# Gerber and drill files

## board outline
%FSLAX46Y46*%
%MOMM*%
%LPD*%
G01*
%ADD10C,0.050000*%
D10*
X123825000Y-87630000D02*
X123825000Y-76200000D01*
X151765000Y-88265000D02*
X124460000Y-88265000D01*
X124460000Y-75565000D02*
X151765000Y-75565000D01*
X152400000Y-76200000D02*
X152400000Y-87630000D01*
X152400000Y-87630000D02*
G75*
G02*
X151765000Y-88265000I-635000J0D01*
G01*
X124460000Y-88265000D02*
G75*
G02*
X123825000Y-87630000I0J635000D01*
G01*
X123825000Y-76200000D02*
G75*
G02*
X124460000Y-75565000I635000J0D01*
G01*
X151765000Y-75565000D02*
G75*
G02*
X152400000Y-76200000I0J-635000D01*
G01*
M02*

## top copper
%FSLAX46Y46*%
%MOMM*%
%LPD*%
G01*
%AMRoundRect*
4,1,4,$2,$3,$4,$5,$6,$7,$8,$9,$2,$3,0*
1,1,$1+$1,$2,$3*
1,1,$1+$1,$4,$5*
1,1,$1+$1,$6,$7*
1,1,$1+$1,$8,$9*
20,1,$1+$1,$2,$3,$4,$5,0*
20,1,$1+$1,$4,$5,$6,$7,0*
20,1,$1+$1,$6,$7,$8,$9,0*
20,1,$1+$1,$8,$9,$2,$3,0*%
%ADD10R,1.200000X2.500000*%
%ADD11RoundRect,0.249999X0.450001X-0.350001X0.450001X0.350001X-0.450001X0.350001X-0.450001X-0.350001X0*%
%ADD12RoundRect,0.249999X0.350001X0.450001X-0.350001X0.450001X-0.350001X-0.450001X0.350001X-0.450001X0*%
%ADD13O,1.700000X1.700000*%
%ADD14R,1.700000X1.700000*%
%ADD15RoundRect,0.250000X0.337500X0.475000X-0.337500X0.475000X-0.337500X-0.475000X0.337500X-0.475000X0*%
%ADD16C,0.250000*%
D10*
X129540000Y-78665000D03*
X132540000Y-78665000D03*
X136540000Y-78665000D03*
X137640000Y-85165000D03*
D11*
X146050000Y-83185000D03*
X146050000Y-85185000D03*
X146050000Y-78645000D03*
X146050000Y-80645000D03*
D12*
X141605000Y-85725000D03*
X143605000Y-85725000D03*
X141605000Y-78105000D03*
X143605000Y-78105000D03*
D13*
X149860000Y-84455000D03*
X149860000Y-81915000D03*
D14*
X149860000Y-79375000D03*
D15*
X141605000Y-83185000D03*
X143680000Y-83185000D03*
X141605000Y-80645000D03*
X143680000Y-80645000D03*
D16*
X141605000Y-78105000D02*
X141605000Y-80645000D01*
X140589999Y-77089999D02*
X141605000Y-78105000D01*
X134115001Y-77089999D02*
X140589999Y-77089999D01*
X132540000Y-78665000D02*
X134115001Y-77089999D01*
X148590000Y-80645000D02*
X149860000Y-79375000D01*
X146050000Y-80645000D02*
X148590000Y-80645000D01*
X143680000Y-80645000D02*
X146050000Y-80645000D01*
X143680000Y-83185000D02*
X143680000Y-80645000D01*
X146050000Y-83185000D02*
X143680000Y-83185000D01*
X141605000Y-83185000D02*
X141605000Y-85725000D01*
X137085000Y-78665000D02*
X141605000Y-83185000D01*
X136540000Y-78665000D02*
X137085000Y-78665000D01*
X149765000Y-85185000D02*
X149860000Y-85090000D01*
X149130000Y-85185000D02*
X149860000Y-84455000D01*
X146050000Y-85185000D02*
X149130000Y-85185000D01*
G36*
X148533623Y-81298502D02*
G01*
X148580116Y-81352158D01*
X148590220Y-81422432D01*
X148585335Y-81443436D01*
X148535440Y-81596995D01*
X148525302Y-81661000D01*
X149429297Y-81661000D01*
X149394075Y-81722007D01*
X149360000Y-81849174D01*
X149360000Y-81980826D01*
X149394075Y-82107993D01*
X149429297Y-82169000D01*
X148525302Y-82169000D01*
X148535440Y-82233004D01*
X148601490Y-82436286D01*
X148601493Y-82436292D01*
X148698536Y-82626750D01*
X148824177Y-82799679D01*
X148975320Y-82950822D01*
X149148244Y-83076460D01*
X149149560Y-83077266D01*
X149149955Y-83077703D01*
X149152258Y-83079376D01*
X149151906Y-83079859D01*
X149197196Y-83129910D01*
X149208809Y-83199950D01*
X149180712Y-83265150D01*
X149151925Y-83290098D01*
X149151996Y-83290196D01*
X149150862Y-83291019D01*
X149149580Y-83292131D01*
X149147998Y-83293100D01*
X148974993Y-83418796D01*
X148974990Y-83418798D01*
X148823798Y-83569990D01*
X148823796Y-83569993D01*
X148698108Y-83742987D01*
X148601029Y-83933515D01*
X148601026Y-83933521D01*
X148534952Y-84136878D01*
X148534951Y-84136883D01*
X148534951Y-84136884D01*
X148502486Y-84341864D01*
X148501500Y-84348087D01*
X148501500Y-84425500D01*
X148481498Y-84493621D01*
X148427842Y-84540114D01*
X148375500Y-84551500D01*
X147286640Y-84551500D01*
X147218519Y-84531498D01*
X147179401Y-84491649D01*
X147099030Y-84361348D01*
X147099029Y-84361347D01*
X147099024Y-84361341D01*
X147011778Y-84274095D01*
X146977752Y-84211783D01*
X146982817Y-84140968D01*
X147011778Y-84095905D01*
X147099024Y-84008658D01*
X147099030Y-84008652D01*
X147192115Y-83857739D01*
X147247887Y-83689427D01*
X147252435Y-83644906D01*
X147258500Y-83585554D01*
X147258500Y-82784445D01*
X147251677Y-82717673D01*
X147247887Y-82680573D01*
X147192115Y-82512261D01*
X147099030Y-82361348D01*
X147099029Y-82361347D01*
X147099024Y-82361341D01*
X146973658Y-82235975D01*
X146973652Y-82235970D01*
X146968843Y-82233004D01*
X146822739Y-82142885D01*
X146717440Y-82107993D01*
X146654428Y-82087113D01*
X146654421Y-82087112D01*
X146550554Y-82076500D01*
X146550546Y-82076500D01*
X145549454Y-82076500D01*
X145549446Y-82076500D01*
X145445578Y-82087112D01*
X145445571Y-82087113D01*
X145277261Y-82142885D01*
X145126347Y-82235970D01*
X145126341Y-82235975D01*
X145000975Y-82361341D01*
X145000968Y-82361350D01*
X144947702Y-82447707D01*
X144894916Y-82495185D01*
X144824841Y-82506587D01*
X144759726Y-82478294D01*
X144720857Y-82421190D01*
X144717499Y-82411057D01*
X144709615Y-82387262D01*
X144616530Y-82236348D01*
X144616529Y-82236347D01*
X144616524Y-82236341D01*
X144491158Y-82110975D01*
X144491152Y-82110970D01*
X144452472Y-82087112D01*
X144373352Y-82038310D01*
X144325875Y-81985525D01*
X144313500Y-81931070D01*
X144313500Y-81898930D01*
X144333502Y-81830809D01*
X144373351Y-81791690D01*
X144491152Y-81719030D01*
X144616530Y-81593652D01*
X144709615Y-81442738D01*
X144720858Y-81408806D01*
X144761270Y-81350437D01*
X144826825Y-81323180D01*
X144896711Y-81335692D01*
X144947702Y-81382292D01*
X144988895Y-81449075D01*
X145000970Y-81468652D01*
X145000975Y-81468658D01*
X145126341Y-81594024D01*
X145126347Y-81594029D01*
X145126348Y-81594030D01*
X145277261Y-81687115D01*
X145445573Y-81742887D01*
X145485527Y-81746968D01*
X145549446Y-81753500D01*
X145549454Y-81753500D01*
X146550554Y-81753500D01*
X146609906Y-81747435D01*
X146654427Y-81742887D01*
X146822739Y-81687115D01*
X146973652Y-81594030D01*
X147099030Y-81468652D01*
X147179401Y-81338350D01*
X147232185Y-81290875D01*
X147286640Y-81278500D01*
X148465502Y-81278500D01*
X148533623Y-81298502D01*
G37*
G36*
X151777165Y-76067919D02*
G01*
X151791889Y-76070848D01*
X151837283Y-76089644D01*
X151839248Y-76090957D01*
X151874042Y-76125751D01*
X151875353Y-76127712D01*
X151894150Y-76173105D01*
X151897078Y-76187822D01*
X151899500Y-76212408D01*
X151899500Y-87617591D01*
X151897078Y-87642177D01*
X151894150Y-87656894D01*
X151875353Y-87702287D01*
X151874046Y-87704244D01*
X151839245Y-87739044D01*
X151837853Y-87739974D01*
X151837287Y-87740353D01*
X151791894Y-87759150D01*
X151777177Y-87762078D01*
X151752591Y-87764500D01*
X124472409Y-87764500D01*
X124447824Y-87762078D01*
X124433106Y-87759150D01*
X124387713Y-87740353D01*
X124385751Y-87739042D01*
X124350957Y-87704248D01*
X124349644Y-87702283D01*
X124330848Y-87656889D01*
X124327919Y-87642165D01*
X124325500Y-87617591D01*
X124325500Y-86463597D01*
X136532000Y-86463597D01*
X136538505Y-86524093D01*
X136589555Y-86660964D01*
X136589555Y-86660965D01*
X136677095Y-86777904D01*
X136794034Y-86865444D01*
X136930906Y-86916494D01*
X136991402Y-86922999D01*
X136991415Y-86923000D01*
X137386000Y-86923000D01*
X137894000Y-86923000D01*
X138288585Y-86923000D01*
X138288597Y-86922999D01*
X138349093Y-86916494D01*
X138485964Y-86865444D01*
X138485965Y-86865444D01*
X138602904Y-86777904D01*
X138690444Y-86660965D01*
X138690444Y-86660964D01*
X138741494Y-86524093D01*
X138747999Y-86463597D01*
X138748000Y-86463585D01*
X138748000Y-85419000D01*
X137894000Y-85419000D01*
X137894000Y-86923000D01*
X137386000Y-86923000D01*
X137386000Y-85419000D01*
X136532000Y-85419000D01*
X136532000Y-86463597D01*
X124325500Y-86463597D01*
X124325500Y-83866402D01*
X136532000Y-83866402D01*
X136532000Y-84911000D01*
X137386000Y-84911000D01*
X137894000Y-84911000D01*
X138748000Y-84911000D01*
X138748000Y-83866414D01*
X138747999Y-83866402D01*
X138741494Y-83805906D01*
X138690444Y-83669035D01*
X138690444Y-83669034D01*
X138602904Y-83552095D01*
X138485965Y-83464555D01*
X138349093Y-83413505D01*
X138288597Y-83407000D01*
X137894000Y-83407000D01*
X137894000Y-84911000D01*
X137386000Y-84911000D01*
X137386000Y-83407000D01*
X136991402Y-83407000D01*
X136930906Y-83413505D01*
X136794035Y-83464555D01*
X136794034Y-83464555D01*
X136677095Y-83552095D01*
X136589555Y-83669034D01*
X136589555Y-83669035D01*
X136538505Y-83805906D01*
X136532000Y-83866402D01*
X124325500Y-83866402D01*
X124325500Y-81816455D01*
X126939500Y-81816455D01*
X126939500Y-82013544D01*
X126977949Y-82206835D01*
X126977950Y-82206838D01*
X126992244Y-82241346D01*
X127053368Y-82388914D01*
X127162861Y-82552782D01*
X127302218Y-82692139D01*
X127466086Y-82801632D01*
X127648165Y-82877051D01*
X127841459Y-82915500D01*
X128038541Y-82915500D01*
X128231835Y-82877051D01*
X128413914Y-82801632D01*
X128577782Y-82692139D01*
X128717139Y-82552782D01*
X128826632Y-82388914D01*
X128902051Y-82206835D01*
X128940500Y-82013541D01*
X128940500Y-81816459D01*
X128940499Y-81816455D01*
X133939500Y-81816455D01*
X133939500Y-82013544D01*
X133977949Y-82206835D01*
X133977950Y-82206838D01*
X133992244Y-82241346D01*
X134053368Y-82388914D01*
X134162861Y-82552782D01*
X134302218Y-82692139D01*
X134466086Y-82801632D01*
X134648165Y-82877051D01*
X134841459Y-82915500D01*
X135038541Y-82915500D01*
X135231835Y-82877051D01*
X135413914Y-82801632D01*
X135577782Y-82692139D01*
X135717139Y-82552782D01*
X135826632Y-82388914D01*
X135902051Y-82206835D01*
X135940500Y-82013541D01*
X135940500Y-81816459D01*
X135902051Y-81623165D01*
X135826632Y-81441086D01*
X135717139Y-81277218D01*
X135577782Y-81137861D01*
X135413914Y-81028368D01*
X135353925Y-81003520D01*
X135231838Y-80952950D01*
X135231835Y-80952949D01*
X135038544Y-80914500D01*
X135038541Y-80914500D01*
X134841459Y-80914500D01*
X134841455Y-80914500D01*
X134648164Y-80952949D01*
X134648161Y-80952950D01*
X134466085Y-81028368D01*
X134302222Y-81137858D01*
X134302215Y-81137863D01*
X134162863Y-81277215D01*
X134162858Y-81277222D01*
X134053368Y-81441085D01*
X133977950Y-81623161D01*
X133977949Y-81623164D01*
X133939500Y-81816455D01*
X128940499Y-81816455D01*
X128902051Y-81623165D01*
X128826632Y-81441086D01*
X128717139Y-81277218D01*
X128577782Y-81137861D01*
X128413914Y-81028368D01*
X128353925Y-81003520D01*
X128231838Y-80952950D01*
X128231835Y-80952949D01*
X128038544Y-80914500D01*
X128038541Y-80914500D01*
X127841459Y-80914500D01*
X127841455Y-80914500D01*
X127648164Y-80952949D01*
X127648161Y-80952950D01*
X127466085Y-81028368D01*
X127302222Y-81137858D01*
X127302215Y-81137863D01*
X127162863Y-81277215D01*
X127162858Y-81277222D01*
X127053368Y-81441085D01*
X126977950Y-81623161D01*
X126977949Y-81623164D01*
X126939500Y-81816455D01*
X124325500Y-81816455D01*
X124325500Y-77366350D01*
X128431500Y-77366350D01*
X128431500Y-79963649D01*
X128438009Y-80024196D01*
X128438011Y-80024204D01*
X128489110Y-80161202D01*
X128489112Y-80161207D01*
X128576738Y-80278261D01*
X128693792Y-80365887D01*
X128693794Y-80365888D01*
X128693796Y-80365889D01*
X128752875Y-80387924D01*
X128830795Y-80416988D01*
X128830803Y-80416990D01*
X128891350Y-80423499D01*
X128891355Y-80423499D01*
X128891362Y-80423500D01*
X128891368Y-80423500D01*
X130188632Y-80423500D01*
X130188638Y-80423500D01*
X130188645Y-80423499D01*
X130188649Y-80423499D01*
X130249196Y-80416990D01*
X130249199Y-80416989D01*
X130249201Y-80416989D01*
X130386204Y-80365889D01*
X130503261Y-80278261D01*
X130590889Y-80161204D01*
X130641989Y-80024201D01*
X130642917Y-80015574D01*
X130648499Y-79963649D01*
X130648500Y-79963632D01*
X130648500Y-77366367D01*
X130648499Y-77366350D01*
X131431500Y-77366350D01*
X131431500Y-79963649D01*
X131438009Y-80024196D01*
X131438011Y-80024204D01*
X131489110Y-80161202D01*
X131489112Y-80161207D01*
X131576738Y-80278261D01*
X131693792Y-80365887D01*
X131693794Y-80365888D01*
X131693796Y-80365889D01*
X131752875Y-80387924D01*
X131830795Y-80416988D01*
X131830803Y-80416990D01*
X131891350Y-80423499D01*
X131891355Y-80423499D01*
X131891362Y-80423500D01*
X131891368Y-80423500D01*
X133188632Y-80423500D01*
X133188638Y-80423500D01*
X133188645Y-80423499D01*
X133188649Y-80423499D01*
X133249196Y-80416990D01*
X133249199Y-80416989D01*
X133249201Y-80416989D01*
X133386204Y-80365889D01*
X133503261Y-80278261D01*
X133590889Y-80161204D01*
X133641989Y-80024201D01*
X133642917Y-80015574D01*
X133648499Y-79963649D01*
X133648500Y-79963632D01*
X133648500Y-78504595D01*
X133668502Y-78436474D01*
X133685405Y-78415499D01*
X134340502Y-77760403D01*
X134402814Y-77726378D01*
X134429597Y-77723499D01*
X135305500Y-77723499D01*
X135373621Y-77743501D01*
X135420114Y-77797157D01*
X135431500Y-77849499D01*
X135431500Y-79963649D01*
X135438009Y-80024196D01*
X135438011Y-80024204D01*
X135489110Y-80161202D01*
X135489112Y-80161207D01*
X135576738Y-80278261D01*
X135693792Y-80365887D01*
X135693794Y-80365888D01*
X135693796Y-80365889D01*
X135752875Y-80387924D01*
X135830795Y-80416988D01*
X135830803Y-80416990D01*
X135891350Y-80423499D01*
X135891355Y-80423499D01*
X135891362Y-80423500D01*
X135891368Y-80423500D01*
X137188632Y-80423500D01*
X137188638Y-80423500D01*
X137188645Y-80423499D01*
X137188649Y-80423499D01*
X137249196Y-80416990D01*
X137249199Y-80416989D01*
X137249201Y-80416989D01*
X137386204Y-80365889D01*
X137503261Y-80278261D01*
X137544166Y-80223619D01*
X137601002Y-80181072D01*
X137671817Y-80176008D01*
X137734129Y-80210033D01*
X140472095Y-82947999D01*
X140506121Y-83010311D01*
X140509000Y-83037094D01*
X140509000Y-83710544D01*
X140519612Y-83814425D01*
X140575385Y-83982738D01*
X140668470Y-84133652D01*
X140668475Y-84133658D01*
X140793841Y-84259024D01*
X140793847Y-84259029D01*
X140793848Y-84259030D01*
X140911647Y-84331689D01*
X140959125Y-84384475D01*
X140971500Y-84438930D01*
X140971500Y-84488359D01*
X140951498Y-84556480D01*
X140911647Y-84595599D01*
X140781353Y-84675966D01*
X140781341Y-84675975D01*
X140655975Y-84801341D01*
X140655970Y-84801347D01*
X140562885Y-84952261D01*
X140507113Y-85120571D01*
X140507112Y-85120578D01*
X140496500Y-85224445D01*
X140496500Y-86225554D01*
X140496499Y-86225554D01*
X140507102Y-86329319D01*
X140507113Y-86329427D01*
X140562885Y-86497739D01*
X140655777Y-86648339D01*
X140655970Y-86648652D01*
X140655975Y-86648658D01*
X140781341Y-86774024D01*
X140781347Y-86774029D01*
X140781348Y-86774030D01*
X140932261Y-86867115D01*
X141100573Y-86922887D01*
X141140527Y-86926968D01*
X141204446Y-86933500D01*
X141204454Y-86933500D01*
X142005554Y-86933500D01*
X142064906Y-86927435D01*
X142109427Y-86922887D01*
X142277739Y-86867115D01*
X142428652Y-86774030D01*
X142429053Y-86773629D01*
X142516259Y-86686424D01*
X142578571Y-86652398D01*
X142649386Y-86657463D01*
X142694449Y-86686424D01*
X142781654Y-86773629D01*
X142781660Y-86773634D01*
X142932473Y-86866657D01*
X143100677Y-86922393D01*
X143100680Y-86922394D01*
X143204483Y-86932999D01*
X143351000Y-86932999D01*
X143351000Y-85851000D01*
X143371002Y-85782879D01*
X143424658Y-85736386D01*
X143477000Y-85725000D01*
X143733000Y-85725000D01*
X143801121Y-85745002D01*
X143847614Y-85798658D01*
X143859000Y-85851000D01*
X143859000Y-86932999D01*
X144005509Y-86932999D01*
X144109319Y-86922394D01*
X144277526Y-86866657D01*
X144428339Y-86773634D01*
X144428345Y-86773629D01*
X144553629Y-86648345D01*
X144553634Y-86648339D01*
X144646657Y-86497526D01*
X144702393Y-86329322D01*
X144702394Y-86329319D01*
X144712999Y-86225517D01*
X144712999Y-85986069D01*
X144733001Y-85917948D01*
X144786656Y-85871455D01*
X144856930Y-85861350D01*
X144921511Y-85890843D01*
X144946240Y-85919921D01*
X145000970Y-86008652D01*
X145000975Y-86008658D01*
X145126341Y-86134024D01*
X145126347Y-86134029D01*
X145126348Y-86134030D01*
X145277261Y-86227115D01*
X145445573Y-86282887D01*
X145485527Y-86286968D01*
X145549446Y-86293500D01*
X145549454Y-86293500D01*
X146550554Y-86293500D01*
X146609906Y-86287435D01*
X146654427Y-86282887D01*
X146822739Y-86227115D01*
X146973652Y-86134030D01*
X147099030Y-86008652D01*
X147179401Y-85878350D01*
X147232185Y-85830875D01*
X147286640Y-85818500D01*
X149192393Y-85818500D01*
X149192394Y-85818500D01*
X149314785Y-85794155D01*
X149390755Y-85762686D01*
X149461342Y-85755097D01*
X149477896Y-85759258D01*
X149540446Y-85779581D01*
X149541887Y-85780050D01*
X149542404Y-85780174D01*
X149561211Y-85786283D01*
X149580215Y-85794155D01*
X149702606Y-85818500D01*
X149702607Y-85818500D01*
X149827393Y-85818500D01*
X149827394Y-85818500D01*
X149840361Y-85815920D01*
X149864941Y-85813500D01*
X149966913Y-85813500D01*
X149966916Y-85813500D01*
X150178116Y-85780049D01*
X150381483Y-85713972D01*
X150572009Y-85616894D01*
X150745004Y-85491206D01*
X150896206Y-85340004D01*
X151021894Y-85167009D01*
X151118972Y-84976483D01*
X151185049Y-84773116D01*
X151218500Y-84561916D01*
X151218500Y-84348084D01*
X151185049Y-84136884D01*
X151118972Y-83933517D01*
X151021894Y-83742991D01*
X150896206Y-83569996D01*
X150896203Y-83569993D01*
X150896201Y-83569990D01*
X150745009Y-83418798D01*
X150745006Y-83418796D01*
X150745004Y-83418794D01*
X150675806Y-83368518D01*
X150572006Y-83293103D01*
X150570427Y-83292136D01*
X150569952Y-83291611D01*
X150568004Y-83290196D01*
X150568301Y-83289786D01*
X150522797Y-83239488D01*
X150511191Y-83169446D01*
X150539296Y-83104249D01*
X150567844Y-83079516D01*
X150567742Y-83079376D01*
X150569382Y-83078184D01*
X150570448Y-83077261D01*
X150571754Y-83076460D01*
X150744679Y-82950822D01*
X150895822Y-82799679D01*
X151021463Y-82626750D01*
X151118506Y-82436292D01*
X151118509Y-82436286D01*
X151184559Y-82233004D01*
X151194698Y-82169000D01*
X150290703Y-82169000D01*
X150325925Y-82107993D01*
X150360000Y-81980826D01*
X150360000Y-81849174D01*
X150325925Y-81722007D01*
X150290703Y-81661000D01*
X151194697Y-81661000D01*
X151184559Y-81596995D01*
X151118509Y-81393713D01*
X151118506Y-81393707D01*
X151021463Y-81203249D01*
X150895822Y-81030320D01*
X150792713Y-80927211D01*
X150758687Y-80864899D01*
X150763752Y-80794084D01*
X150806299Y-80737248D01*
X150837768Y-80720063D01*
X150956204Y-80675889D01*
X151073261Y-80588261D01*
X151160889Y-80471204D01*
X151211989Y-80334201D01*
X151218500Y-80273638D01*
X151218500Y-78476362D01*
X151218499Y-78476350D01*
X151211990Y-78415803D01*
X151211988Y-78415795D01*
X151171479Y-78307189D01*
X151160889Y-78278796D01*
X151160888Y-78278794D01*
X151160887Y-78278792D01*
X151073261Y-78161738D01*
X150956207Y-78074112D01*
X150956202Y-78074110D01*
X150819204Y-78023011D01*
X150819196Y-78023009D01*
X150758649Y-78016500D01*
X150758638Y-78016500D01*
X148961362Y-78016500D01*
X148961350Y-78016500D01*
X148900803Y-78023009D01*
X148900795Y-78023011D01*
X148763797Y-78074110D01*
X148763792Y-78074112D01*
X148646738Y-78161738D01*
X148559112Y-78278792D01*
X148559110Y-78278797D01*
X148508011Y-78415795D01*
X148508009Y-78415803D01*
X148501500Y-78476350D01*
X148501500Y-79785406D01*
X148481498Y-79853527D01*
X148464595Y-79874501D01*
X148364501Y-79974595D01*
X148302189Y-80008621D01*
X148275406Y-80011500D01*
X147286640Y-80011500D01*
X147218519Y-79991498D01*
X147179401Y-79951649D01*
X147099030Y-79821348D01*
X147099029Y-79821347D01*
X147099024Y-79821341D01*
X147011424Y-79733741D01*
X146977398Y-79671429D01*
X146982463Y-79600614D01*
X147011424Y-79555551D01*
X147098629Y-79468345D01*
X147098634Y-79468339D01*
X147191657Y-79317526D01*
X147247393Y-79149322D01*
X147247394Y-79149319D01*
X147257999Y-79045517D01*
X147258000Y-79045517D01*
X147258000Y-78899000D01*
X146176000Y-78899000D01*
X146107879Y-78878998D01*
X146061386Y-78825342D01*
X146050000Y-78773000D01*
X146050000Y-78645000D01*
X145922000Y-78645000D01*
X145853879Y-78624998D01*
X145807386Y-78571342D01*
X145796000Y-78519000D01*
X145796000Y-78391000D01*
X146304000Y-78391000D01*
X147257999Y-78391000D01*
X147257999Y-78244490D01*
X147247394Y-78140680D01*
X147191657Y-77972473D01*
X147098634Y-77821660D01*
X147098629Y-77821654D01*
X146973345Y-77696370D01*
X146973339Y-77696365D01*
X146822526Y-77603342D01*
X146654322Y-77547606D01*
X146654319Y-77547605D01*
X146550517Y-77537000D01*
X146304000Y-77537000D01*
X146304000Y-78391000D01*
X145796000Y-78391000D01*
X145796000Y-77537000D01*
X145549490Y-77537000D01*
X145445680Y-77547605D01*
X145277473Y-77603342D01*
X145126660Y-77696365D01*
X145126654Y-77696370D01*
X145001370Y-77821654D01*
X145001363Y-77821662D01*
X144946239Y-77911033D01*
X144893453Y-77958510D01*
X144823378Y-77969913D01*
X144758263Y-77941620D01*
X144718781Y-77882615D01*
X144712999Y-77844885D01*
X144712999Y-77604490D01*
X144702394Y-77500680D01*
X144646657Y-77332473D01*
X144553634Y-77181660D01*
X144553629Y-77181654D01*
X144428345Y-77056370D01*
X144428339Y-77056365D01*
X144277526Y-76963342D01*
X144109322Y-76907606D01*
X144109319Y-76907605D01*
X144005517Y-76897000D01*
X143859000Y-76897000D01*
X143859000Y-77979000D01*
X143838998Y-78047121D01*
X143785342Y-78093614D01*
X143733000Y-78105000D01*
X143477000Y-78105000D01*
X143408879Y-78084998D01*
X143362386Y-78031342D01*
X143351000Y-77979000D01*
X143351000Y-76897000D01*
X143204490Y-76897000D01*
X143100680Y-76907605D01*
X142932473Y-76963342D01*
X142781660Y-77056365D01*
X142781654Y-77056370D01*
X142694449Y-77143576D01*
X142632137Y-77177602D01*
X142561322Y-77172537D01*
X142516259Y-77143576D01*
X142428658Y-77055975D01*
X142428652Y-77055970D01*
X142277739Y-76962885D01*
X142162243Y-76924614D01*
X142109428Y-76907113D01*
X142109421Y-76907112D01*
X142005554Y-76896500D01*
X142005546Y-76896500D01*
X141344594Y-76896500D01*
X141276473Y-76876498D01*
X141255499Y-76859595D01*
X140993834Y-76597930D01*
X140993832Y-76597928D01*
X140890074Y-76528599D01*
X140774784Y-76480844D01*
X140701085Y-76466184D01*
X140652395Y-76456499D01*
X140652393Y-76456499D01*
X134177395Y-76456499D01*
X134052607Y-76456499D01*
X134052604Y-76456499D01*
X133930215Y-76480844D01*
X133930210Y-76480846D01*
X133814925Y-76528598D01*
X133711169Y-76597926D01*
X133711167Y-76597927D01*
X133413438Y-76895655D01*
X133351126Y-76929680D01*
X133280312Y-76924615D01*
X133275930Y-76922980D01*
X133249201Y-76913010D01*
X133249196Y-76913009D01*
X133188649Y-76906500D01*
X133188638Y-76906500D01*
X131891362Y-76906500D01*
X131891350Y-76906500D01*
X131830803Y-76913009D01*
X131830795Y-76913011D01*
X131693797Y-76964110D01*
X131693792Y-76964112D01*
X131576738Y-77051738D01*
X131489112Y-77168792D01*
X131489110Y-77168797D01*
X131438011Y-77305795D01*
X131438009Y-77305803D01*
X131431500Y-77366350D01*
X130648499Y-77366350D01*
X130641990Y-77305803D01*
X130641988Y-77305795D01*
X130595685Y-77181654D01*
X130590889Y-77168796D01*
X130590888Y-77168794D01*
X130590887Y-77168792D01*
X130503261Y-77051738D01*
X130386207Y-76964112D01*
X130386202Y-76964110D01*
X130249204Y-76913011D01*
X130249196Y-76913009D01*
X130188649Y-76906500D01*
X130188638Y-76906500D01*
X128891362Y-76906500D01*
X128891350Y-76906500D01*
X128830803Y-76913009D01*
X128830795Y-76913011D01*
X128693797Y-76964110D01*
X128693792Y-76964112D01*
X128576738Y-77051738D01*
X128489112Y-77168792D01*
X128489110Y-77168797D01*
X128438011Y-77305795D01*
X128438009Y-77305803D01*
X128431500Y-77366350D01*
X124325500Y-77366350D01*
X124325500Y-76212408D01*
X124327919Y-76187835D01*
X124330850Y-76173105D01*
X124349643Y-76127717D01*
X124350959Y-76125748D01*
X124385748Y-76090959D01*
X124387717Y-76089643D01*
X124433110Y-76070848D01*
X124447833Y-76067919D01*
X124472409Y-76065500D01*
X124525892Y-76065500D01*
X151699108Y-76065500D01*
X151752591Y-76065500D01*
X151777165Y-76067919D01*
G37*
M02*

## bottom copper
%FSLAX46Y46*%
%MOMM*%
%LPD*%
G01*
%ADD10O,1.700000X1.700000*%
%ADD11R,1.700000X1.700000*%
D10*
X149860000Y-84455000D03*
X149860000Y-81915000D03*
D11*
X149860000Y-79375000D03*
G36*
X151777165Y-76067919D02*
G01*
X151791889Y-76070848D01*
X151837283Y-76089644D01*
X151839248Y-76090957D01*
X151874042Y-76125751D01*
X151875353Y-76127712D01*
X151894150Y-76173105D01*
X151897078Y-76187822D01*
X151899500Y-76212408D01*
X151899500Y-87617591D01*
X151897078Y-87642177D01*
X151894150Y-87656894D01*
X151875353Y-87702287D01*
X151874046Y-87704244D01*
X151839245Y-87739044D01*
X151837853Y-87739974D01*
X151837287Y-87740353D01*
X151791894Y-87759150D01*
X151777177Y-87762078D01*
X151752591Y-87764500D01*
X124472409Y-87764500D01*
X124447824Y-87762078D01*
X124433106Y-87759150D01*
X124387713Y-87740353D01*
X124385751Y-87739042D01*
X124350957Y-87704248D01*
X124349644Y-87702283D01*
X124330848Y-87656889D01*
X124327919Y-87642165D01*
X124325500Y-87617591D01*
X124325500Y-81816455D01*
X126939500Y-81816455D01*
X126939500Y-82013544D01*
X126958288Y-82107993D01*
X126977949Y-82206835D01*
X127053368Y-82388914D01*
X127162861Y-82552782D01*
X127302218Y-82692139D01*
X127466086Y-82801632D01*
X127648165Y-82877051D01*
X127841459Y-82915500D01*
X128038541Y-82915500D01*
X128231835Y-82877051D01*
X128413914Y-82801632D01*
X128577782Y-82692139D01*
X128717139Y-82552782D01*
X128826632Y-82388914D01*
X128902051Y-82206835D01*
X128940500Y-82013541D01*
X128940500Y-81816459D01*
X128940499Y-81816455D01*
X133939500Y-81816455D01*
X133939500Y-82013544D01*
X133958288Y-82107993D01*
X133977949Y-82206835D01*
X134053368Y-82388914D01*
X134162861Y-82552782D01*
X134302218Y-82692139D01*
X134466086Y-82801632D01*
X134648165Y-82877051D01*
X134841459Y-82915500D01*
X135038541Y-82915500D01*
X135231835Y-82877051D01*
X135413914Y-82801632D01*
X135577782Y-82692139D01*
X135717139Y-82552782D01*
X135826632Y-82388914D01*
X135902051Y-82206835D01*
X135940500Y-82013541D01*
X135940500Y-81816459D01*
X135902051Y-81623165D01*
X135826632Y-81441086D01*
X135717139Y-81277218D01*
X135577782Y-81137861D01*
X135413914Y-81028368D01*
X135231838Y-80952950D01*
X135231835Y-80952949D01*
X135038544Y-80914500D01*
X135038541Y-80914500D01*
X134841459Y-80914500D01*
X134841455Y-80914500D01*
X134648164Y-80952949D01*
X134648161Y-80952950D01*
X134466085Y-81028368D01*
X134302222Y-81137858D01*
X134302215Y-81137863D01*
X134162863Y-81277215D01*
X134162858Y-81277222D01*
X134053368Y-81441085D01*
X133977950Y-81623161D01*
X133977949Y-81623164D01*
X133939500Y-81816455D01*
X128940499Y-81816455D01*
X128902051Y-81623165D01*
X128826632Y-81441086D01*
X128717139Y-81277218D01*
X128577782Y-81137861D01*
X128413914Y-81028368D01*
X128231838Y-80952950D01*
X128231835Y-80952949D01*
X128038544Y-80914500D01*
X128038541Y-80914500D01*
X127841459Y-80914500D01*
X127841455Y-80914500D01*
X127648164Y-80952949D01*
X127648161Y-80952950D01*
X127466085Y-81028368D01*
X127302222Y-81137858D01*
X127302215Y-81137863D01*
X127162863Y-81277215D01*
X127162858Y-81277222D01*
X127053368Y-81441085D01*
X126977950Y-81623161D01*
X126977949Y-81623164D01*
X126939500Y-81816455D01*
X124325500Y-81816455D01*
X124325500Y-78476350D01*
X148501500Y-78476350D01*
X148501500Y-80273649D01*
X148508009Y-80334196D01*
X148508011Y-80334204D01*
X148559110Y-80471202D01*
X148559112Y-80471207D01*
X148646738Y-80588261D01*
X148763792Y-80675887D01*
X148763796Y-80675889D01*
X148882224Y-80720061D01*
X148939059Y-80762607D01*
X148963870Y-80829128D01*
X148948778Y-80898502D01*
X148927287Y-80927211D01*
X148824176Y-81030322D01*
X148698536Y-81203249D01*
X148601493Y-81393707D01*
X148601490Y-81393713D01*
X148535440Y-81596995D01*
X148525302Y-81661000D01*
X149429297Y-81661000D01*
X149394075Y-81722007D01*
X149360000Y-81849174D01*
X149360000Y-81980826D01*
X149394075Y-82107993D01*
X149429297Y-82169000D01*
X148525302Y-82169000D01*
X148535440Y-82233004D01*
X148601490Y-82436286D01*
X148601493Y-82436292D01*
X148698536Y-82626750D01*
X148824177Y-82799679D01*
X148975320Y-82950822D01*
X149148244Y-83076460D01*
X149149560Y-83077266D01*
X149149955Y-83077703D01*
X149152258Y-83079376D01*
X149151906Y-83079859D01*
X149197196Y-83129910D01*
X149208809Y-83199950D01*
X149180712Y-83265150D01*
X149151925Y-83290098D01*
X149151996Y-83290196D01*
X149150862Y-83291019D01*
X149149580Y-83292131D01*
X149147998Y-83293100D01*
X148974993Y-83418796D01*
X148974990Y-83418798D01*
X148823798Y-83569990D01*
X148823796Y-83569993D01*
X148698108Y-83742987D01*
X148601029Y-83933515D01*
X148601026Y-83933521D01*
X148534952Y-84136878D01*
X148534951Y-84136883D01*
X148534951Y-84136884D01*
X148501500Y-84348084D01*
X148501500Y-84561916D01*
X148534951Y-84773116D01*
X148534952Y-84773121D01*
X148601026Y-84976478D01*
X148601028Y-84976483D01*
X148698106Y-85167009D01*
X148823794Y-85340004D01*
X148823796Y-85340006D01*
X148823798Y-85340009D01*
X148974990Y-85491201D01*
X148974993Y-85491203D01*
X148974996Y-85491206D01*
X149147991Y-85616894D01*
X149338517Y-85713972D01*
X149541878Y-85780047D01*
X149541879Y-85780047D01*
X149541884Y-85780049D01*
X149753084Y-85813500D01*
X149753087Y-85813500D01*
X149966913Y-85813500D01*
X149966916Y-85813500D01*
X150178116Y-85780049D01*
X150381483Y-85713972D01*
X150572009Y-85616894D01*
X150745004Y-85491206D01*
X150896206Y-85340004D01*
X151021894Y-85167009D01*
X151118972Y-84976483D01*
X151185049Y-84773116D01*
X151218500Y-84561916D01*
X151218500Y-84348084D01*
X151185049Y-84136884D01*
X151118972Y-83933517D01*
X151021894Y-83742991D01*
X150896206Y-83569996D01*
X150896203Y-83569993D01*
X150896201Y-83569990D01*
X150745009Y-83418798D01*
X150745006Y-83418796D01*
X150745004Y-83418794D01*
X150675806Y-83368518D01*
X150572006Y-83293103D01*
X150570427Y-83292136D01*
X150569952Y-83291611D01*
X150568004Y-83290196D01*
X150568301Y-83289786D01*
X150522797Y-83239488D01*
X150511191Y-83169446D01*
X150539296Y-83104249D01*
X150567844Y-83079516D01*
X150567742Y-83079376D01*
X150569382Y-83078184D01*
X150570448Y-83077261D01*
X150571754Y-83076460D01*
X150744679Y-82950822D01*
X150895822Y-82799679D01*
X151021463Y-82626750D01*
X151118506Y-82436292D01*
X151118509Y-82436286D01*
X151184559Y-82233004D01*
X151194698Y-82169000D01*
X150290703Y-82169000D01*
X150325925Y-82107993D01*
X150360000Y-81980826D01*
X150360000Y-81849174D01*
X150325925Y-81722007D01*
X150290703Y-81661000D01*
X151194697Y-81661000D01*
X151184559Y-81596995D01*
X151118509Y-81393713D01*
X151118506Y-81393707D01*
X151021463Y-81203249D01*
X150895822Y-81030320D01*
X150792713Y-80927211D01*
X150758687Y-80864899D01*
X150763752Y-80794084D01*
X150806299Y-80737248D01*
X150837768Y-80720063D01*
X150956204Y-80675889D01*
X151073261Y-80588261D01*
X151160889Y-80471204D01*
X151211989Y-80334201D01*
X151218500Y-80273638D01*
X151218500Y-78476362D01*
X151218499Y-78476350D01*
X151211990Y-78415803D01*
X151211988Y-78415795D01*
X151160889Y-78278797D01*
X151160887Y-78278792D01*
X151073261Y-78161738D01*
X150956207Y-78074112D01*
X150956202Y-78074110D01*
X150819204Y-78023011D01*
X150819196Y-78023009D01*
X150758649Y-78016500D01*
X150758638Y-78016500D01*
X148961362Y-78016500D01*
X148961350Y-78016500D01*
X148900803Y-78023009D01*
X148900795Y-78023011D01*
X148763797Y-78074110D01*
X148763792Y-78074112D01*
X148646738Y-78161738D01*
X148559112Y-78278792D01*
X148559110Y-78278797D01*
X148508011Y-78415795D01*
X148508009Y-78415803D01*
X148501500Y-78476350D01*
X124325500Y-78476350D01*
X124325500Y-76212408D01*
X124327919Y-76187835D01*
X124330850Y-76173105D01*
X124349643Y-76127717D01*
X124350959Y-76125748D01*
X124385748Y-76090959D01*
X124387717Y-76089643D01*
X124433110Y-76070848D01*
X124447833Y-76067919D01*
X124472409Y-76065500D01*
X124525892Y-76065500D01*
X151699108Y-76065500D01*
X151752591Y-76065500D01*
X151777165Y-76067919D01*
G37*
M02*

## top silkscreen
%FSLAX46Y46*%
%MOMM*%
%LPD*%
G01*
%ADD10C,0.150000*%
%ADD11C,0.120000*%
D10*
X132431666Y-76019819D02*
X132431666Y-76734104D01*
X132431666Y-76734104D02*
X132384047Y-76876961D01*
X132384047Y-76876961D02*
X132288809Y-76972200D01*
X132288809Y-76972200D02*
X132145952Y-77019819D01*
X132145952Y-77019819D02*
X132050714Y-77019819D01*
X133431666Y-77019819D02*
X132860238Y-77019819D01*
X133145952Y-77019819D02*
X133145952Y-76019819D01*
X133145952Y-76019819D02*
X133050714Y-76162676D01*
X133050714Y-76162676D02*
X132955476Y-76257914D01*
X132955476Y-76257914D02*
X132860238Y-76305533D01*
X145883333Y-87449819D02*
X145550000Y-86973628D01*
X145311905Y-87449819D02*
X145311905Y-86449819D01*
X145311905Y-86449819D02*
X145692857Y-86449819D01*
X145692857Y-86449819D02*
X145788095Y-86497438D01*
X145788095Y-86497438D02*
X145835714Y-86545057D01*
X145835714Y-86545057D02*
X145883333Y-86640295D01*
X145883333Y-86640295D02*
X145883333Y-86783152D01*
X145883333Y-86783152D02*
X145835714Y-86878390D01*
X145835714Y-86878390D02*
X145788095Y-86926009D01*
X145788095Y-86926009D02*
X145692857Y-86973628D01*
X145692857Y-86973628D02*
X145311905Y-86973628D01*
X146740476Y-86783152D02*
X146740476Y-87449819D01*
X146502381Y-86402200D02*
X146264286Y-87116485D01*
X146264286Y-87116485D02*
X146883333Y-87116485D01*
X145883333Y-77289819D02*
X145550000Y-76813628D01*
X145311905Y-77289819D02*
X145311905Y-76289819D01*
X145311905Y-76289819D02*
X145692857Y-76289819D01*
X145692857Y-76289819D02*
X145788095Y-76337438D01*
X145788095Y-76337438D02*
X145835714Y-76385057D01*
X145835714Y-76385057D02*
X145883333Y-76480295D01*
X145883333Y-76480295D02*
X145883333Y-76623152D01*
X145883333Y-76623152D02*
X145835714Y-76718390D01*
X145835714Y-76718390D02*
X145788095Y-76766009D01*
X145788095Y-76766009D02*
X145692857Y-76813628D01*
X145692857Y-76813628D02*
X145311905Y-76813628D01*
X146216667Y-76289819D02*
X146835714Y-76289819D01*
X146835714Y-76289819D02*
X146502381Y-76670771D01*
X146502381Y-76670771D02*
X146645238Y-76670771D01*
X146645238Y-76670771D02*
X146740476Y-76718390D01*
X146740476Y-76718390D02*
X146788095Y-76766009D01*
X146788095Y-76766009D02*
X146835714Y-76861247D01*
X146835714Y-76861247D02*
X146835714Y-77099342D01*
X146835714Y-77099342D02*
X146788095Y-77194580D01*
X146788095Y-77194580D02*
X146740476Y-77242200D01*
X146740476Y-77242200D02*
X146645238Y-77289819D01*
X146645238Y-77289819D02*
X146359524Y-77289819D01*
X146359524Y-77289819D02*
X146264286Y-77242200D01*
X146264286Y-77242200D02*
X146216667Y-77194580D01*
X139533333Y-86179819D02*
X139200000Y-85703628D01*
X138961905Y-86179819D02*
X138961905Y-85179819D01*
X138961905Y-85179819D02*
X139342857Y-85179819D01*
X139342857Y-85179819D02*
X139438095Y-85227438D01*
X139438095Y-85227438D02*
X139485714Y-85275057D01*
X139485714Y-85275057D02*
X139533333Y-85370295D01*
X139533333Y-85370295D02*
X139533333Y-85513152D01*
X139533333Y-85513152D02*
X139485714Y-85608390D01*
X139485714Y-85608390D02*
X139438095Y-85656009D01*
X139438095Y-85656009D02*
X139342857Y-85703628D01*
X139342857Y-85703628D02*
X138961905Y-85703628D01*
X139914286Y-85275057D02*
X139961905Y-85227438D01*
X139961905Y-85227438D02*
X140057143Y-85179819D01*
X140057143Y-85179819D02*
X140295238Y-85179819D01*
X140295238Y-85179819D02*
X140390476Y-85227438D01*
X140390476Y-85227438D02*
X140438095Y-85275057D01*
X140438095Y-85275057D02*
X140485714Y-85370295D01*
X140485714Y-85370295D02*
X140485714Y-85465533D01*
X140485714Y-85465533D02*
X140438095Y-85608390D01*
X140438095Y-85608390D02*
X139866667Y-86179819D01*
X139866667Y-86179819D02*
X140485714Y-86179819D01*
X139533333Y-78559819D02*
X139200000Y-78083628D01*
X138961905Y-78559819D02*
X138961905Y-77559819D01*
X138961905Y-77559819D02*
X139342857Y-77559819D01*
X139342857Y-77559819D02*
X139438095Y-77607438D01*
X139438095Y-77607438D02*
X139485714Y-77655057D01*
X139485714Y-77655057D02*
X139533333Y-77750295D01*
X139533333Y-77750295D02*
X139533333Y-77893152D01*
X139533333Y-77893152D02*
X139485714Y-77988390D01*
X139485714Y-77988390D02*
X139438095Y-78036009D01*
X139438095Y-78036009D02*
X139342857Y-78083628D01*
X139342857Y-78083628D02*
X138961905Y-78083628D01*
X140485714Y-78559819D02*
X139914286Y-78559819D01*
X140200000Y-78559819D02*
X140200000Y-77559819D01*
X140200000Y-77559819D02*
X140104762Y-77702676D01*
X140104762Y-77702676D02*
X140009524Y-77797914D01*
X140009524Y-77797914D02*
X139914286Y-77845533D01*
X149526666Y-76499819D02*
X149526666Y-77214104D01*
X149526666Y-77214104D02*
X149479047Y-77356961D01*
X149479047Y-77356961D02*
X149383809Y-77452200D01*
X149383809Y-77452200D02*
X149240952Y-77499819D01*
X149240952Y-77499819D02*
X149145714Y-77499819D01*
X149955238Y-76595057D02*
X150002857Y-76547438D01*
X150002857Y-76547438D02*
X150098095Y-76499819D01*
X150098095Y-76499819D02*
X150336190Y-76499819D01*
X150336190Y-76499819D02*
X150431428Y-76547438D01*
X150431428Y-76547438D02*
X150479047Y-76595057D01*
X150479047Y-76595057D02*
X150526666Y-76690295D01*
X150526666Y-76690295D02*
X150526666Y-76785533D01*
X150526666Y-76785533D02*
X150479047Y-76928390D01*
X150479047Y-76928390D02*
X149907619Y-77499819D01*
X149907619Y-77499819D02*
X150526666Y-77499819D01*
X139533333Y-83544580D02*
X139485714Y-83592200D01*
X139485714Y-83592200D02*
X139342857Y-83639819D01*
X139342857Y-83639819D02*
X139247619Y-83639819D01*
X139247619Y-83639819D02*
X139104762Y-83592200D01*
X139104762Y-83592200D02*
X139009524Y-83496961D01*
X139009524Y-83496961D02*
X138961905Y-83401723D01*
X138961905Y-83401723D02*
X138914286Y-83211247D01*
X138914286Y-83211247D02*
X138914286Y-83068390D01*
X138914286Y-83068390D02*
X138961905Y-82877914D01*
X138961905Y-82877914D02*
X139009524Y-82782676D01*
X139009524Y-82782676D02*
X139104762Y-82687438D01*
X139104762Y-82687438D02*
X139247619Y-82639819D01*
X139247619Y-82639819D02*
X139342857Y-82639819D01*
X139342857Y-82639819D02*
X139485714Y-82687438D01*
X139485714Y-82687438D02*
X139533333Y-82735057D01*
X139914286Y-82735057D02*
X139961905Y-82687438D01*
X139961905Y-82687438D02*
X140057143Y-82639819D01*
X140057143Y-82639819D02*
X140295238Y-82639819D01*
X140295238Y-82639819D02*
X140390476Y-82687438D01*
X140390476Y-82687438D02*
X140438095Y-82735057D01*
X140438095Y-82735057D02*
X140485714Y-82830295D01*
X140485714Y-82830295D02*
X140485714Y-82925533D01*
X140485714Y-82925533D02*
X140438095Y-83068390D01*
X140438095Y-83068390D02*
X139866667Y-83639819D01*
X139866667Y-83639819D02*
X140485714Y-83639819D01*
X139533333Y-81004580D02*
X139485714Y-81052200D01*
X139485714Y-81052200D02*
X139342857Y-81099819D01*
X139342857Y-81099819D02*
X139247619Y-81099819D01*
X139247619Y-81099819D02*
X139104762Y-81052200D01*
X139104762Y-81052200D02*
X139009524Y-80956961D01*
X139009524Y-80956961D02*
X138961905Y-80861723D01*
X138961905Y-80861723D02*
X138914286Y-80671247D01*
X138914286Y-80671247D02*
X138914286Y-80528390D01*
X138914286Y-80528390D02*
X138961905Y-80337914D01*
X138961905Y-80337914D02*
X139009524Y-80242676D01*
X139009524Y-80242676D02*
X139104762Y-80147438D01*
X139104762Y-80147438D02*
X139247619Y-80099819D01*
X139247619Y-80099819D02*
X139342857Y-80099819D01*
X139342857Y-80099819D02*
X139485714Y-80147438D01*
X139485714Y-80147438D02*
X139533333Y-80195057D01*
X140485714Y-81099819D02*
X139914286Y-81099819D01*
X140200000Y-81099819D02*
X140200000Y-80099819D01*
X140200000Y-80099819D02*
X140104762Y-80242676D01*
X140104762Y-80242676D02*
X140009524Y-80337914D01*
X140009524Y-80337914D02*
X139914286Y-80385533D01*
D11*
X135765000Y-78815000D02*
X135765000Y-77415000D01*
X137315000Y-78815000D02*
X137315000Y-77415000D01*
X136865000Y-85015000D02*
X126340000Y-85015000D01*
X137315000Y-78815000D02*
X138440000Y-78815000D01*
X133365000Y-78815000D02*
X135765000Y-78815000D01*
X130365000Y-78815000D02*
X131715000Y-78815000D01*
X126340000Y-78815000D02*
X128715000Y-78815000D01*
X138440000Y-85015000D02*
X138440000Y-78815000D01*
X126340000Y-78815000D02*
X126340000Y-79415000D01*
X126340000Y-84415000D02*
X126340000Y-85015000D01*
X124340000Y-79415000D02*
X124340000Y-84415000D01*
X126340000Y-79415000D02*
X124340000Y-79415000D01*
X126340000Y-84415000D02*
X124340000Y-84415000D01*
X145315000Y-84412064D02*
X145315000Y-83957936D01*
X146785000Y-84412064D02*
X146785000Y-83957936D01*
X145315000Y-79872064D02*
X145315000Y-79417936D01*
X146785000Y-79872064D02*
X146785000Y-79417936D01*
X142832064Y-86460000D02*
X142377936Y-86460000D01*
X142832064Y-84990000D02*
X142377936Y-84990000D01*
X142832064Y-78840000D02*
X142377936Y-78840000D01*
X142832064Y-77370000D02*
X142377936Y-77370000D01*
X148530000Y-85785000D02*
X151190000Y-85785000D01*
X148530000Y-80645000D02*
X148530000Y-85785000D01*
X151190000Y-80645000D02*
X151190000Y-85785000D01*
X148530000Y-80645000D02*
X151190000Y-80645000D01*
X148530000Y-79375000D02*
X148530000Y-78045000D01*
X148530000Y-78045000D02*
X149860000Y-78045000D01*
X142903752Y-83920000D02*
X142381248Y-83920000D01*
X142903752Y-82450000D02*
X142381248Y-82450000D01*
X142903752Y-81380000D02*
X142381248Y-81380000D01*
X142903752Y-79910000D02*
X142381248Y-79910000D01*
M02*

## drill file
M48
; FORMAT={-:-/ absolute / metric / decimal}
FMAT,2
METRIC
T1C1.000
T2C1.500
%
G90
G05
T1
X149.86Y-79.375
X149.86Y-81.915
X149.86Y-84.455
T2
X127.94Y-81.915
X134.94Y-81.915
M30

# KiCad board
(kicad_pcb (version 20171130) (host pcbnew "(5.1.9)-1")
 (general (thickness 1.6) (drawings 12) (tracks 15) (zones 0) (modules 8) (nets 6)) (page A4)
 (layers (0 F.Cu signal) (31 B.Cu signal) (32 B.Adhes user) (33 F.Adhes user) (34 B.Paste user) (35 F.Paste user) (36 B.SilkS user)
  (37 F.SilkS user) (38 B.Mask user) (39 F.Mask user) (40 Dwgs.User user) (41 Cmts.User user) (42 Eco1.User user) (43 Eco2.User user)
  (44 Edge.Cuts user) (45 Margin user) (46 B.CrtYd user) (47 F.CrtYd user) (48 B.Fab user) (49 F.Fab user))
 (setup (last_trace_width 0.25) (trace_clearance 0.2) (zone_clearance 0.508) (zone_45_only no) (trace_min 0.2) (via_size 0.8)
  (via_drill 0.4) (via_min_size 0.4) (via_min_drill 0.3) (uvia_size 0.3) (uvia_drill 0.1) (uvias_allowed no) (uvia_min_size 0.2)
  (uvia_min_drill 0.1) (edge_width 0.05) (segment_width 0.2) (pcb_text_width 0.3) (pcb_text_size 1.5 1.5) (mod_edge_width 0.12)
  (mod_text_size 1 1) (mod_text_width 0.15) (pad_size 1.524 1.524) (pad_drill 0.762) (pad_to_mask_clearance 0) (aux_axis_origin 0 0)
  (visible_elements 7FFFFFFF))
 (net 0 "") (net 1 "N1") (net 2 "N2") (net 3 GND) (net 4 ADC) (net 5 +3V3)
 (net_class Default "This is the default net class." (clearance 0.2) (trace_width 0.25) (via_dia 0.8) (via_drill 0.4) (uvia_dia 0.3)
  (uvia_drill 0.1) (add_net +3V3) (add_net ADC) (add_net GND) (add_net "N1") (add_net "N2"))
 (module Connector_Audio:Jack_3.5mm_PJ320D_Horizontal (layer F.Cu) (at 132.715 81.915)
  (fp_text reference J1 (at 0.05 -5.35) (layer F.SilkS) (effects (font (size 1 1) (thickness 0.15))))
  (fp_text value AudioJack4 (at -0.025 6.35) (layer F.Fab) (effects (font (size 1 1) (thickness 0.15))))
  (fp_line (start 3.05 -3.1) (end 3.05 -4.5) (layer F.SilkS) (width 0.12))
  (fp_line (start 4.6 -3.1) (end 4.6 -4.5) (layer F.SilkS) (width 0.12))
  (fp_line (start 4.15 3.1) (end -6.375 3.1) (layer F.SilkS) (width 0.12))
  (fp_line (start 4.6 -3.1) (end 5.725 -3.1) (layer F.SilkS) (width 0.12))
  (fp_line (start 0.65 -3.1) (end 3.05 -3.1) (layer F.SilkS) (width 0.12))
  (fp_line (start -2.35 -3.1) (end -1 -3.1) (layer F.SilkS) (width 0.12))
  (fp_line (start -6.375 -3.1) (end -4 -3.1) (layer F.SilkS) (width 0.12))
  (fp_line (start 5.725 3.1) (end 5.725 -3.1) (layer F.SilkS) (width 0.12))
  (fp_line (start -6.375 -3.1) (end -6.375 -2.5) (layer F.SilkS) (width 0.12))
  (fp_line (start -6.375 2.5) (end -6.375 3.1) (layer F.SilkS) (width 0.12))
  (fp_line (start -8.375 -2.5) (end -8.375 2.5) (layer F.SilkS) (width 0.12))
  (fp_line (start -6.375 -2.5) (end -8.375 -2.5) (layer F.SilkS) (width 0.12))
  (fp_line (start -6.375 2.5) (end -8.375 2.5) (layer F.SilkS) (width 0.12))
  (pad "" np_thru_hole circle (at 2.225 0) (size 1.5 1.5) (drill 1.5) (layers *.Cu *.Mask))
  (pad "" np_thru_hole circle (at -4.775 0) (size 1.5 1.5) (drill 1.5) (layers *.Cu *.Mask))
  (pad R2 smd rect (at -3.175 -3.25) (size 1.2 2.5) (layers F.Cu F.Paste F.Mask))
  (pad R1 smd rect (at -0.175 -3.25) (size 1.2 2.5) (layers F.Cu F.Paste F.Mask) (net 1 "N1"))
  (pad T smd rect (at 3.825 -3.25) (size 1.2 2.5) (layers F.Cu F.Paste F.Mask) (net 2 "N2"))
  (pad S smd rect (at 4.925 3.25) (size 1.2 2.5) (layers F.Cu F.Paste F.Mask) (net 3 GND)))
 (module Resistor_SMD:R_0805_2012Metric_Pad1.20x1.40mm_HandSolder (layer F.Cu) (at 146.05 84.185 90)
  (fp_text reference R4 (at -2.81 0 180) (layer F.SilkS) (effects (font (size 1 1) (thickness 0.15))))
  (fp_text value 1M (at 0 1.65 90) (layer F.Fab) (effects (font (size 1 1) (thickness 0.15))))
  (fp_line (start -0.227064 -0.735) (end 0.227064 -0.735) (layer F.SilkS) (width 0.12))
  (fp_line (start -0.227064 0.735) (end 0.227064 0.735) (layer F.SilkS) (width 0.12))
  (pad 2 smd roundrect (at 1 0 90) (size 1.2 1.4) (layers F.Cu F.Paste F.Mask) (roundrect_rratio 0.2083325) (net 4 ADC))
  (pad 1 smd roundrect (at -1 0 90) (size 1.2 1.4) (layers F.Cu F.Paste F.Mask) (roundrect_rratio 0.2083325) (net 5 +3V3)))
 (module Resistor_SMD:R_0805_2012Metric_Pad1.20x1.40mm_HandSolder (layer F.Cu) (at 146.05 79.645 90)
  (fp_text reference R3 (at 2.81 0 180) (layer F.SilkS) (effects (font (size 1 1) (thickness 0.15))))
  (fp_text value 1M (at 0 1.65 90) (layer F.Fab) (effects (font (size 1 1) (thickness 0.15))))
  (fp_line (start -0.227064 -0.735) (end 0.227064 -0.735) (layer F.SilkS) (width 0.12))
  (fp_line (start -0.227064 0.735) (end 0.227064 0.735) (layer F.SilkS) (width 0.12))
  (pad 2 smd roundrect (at 1 0 90) (size 1.2 1.4) (layers F.Cu F.Paste F.Mask) (roundrect_rratio 0.2083325) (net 3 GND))
  (pad 1 smd roundrect (at -1 0 90) (size 1.2 1.4) (layers F.Cu F.Paste F.Mask) (roundrect_rratio 0.2083325) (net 4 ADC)))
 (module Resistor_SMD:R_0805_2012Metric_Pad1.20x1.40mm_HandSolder (layer F.Cu) (at 142.605 85.725 180)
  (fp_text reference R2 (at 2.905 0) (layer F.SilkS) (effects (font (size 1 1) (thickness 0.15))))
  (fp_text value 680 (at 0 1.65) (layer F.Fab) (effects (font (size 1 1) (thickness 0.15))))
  (fp_line (start -0.227064 -0.735) (end 0.227064 -0.735) (layer F.SilkS) (width 0.12))
  (fp_line (start -0.227064 0.735) (end 0.227064 0.735) (layer F.SilkS) (width 0.12))
  (pad 2 smd roundrect (at 1 0 180) (size 1.2 1.4) (layers F.Cu F.Paste F.Mask) (roundrect_rratio 0.2083325) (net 2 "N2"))
  (pad 1 smd roundrect (at -1 0 180) (size 1.2 1.4) (layers F.Cu F.Paste F.Mask) (roundrect_rratio 0.2083325) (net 3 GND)))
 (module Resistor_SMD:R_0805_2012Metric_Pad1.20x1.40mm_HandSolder (layer F.Cu) (at 142.605 78.105 180)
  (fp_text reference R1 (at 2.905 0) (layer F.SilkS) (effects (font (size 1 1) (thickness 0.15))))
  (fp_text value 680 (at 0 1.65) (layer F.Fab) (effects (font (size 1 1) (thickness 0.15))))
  (fp_line (start -0.227064 -0.735) (end 0.227064 -0.735) (layer F.SilkS) (width 0.12))
  (fp_line (start -0.227064 0.735) (end 0.227064 0.735) (layer F.SilkS) (width 0.12))
  (pad 2 smd roundrect (at 1 0 180) (size 1.2 1.4) (layers F.Cu F.Paste F.Mask) (roundrect_rratio 0.2083325) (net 1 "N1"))
  (pad 1 smd roundrect (at -1 0 180) (size 1.2 1.4) (layers F.Cu F.Paste F.Mask) (roundrect_rratio 0.2083325) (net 3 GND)))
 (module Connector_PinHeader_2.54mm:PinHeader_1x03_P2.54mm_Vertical (layer F.Cu) (at 149.86 79.375)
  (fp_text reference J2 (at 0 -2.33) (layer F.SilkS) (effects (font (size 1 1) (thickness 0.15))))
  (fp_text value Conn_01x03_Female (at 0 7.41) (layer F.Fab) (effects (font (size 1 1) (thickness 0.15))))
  (fp_line (start -1.33 6.41) (end 1.33 6.41) (layer F.SilkS) (width 0.12))
  (fp_line (start -1.33 1.27) (end -1.33 6.41) (layer F.SilkS) (width 0.12))
  (fp_line (start 1.33 1.27) (end 1.33 6.41) (layer F.SilkS) (width 0.12))
  (fp_line (start -1.33 1.27) (end 1.33 1.27) (layer F.SilkS) (width 0.12))
  (fp_line (start -1.33 0) (end -1.33 -1.33) (layer F.SilkS) (width 0.12))
  (fp_line (start -1.33 -1.33) (end 0 -1.33) (layer F.SilkS) (width 0.12))
  (pad 3 thru_hole oval (at 0 5.08) (size 1.7 1.7) (drill 1) (layers *.Cu *.Mask) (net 5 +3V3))
  (pad 2 thru_hole oval (at 0 2.54) (size 1.7 1.7) (drill 1) (layers *.Cu *.Mask) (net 3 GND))
  (pad 1 thru_hole rect (at 0 0) (size 1.7 1.7) (drill 1) (layers *.Cu *.Mask) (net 4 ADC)))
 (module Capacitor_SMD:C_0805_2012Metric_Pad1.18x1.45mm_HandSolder (layer F.Cu) (at 142.6425 83.185 180)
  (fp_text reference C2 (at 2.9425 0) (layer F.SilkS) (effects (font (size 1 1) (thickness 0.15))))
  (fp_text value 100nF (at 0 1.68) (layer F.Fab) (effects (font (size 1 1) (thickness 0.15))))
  (fp_line (start -0.261252 -0.735) (end 0.261252 -0.735) (layer F.SilkS) (width 0.12))
  (fp_line (start -0.261252 0.735) (end 0.261252 0.735) (layer F.SilkS) (width 0.12))
  (pad 2 smd roundrect (at 1.0375 0 180) (size 1.175 1.45) (layers F.Cu F.Paste F.Mask) (roundrect_rratio 0.2127659574468085) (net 2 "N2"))
  (pad 1 smd roundrect (at -1.0375 0 180) (size 1.175 1.45) (layers F.Cu F.Paste F.Mask) (roundrect_rratio 0.2127659574468085) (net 4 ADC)))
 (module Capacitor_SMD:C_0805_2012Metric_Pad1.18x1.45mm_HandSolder (layer F.Cu) (at 142.6425 80.645 180)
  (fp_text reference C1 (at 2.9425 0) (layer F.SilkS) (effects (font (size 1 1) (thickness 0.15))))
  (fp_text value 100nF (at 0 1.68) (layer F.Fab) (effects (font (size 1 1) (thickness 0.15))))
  (fp_line (start -0.261252 -0.735) (end 0.261252 -0.735) (layer F.SilkS) (width 0.12))
  (fp_line (start -0.261252 0.735) (end 0.261252 0.735) (layer F.SilkS) (width 0.12))
  (pad 2 smd roundrect (at 1.0375 0 180) (size 1.175 1.45) (layers F.Cu F.Paste F.Mask) (roundrect_rratio 0.2127659574468085) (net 1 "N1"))
  (pad 1 smd roundrect (at -1.0375 0 180) (size 1.175 1.45) (layers F.Cu F.Paste F.Mask) (roundrect_rratio 0.2127659574468085) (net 4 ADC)))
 (gr_line (start 123.825 87.63) (end 123.825 76.2) (layer Edge.Cuts) (width 0.05))
 (gr_line (start 151.765 88.265) (end 124.46 88.265) (layer Edge.Cuts) (width 0.05))
 (gr_line (start 124.46 75.565) (end 151.765 75.565) (layer Edge.Cuts) (width 0.05))
 (gr_line (start 152.4 76.2) (end 152.4 87.63) (layer Edge.Cuts) (width 0.05))
 (gr_arc (start 151.765 87.63) (end 151.765 88.265) (angle -90) (layer Edge.Cuts) (width 0.05))
 (gr_arc (start 124.46 87.63) (end 123.825 87.63) (angle -90) (layer Edge.Cuts) (width 0.05))
 (gr_arc (start 124.46 76.2) (end 124.46 75.565) (angle -90) (layer Edge.Cuts) (width 0.05))
 (gr_arc (start 151.765 76.2) (end 152.4 76.2) (angle -90) (layer Edge.Cuts) (width 0.05))
 (segment (start 141.605 78.105) (end 141.605 80.645) (width 0.25) (layer F.Cu) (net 1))
 (segment (start 140.589999 77.089999) (end 141.605 78.105) (width 0.25) (layer F.Cu) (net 1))
 (segment (start 134.115001 77.089999) (end 140.589999 77.089999) (width 0.25) (layer F.Cu) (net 1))
 (segment (start 132.54 78.665) (end 134.115001 77.089999) (width 0.25) (layer F.Cu) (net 1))
 (segment (start 148.59 80.645) (end 149.86 79.375) (width 0.25) (layer F.Cu) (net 4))
 (segment (start 146.05 80.645) (end 148.59 80.645) (width 0.25) (layer F.Cu) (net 4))
 (segment (start 143.68 80.645) (end 146.05 80.645) (width 0.25) (layer F.Cu) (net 4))
 (segment (start 143.68 83.185) (end 143.68 80.645) (width 0.25) (layer F.Cu) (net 4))
 (segment (start 146.05 83.185) (end 143.68 83.185) (width 0.25) (layer F.Cu) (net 4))
 (segment (start 141.605 83.185) (end 141.605 85.725) (width 0.25) (layer F.Cu) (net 2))
 (segment (start 137.085 78.665) (end 141.605 83.185) (width 0.25) (layer F.Cu) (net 2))
 (segment (start 136.54 78.665) (end 137.085 78.665) (width 0.25) (layer F.Cu) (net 2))
 (segment (start 149.765 85.185) (end 149.86 85.09) (width 0.25) (layer F.Cu) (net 5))
 (segment (start 149.13 85.185) (end 149.86 84.455) (width 0.25) (layer F.Cu) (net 5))
 (segment (start 146.05 85.185) (end 149.13 85.185) (width 0.25) (layer F.Cu) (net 5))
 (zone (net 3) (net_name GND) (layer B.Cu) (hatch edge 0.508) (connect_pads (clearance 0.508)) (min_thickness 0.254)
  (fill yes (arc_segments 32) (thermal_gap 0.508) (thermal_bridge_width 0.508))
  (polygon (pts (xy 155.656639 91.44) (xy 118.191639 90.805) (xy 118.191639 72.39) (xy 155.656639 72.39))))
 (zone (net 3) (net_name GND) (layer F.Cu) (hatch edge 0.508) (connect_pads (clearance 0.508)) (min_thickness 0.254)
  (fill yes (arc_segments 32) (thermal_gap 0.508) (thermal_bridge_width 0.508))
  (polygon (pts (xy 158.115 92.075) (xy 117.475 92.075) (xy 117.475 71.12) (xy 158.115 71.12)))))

